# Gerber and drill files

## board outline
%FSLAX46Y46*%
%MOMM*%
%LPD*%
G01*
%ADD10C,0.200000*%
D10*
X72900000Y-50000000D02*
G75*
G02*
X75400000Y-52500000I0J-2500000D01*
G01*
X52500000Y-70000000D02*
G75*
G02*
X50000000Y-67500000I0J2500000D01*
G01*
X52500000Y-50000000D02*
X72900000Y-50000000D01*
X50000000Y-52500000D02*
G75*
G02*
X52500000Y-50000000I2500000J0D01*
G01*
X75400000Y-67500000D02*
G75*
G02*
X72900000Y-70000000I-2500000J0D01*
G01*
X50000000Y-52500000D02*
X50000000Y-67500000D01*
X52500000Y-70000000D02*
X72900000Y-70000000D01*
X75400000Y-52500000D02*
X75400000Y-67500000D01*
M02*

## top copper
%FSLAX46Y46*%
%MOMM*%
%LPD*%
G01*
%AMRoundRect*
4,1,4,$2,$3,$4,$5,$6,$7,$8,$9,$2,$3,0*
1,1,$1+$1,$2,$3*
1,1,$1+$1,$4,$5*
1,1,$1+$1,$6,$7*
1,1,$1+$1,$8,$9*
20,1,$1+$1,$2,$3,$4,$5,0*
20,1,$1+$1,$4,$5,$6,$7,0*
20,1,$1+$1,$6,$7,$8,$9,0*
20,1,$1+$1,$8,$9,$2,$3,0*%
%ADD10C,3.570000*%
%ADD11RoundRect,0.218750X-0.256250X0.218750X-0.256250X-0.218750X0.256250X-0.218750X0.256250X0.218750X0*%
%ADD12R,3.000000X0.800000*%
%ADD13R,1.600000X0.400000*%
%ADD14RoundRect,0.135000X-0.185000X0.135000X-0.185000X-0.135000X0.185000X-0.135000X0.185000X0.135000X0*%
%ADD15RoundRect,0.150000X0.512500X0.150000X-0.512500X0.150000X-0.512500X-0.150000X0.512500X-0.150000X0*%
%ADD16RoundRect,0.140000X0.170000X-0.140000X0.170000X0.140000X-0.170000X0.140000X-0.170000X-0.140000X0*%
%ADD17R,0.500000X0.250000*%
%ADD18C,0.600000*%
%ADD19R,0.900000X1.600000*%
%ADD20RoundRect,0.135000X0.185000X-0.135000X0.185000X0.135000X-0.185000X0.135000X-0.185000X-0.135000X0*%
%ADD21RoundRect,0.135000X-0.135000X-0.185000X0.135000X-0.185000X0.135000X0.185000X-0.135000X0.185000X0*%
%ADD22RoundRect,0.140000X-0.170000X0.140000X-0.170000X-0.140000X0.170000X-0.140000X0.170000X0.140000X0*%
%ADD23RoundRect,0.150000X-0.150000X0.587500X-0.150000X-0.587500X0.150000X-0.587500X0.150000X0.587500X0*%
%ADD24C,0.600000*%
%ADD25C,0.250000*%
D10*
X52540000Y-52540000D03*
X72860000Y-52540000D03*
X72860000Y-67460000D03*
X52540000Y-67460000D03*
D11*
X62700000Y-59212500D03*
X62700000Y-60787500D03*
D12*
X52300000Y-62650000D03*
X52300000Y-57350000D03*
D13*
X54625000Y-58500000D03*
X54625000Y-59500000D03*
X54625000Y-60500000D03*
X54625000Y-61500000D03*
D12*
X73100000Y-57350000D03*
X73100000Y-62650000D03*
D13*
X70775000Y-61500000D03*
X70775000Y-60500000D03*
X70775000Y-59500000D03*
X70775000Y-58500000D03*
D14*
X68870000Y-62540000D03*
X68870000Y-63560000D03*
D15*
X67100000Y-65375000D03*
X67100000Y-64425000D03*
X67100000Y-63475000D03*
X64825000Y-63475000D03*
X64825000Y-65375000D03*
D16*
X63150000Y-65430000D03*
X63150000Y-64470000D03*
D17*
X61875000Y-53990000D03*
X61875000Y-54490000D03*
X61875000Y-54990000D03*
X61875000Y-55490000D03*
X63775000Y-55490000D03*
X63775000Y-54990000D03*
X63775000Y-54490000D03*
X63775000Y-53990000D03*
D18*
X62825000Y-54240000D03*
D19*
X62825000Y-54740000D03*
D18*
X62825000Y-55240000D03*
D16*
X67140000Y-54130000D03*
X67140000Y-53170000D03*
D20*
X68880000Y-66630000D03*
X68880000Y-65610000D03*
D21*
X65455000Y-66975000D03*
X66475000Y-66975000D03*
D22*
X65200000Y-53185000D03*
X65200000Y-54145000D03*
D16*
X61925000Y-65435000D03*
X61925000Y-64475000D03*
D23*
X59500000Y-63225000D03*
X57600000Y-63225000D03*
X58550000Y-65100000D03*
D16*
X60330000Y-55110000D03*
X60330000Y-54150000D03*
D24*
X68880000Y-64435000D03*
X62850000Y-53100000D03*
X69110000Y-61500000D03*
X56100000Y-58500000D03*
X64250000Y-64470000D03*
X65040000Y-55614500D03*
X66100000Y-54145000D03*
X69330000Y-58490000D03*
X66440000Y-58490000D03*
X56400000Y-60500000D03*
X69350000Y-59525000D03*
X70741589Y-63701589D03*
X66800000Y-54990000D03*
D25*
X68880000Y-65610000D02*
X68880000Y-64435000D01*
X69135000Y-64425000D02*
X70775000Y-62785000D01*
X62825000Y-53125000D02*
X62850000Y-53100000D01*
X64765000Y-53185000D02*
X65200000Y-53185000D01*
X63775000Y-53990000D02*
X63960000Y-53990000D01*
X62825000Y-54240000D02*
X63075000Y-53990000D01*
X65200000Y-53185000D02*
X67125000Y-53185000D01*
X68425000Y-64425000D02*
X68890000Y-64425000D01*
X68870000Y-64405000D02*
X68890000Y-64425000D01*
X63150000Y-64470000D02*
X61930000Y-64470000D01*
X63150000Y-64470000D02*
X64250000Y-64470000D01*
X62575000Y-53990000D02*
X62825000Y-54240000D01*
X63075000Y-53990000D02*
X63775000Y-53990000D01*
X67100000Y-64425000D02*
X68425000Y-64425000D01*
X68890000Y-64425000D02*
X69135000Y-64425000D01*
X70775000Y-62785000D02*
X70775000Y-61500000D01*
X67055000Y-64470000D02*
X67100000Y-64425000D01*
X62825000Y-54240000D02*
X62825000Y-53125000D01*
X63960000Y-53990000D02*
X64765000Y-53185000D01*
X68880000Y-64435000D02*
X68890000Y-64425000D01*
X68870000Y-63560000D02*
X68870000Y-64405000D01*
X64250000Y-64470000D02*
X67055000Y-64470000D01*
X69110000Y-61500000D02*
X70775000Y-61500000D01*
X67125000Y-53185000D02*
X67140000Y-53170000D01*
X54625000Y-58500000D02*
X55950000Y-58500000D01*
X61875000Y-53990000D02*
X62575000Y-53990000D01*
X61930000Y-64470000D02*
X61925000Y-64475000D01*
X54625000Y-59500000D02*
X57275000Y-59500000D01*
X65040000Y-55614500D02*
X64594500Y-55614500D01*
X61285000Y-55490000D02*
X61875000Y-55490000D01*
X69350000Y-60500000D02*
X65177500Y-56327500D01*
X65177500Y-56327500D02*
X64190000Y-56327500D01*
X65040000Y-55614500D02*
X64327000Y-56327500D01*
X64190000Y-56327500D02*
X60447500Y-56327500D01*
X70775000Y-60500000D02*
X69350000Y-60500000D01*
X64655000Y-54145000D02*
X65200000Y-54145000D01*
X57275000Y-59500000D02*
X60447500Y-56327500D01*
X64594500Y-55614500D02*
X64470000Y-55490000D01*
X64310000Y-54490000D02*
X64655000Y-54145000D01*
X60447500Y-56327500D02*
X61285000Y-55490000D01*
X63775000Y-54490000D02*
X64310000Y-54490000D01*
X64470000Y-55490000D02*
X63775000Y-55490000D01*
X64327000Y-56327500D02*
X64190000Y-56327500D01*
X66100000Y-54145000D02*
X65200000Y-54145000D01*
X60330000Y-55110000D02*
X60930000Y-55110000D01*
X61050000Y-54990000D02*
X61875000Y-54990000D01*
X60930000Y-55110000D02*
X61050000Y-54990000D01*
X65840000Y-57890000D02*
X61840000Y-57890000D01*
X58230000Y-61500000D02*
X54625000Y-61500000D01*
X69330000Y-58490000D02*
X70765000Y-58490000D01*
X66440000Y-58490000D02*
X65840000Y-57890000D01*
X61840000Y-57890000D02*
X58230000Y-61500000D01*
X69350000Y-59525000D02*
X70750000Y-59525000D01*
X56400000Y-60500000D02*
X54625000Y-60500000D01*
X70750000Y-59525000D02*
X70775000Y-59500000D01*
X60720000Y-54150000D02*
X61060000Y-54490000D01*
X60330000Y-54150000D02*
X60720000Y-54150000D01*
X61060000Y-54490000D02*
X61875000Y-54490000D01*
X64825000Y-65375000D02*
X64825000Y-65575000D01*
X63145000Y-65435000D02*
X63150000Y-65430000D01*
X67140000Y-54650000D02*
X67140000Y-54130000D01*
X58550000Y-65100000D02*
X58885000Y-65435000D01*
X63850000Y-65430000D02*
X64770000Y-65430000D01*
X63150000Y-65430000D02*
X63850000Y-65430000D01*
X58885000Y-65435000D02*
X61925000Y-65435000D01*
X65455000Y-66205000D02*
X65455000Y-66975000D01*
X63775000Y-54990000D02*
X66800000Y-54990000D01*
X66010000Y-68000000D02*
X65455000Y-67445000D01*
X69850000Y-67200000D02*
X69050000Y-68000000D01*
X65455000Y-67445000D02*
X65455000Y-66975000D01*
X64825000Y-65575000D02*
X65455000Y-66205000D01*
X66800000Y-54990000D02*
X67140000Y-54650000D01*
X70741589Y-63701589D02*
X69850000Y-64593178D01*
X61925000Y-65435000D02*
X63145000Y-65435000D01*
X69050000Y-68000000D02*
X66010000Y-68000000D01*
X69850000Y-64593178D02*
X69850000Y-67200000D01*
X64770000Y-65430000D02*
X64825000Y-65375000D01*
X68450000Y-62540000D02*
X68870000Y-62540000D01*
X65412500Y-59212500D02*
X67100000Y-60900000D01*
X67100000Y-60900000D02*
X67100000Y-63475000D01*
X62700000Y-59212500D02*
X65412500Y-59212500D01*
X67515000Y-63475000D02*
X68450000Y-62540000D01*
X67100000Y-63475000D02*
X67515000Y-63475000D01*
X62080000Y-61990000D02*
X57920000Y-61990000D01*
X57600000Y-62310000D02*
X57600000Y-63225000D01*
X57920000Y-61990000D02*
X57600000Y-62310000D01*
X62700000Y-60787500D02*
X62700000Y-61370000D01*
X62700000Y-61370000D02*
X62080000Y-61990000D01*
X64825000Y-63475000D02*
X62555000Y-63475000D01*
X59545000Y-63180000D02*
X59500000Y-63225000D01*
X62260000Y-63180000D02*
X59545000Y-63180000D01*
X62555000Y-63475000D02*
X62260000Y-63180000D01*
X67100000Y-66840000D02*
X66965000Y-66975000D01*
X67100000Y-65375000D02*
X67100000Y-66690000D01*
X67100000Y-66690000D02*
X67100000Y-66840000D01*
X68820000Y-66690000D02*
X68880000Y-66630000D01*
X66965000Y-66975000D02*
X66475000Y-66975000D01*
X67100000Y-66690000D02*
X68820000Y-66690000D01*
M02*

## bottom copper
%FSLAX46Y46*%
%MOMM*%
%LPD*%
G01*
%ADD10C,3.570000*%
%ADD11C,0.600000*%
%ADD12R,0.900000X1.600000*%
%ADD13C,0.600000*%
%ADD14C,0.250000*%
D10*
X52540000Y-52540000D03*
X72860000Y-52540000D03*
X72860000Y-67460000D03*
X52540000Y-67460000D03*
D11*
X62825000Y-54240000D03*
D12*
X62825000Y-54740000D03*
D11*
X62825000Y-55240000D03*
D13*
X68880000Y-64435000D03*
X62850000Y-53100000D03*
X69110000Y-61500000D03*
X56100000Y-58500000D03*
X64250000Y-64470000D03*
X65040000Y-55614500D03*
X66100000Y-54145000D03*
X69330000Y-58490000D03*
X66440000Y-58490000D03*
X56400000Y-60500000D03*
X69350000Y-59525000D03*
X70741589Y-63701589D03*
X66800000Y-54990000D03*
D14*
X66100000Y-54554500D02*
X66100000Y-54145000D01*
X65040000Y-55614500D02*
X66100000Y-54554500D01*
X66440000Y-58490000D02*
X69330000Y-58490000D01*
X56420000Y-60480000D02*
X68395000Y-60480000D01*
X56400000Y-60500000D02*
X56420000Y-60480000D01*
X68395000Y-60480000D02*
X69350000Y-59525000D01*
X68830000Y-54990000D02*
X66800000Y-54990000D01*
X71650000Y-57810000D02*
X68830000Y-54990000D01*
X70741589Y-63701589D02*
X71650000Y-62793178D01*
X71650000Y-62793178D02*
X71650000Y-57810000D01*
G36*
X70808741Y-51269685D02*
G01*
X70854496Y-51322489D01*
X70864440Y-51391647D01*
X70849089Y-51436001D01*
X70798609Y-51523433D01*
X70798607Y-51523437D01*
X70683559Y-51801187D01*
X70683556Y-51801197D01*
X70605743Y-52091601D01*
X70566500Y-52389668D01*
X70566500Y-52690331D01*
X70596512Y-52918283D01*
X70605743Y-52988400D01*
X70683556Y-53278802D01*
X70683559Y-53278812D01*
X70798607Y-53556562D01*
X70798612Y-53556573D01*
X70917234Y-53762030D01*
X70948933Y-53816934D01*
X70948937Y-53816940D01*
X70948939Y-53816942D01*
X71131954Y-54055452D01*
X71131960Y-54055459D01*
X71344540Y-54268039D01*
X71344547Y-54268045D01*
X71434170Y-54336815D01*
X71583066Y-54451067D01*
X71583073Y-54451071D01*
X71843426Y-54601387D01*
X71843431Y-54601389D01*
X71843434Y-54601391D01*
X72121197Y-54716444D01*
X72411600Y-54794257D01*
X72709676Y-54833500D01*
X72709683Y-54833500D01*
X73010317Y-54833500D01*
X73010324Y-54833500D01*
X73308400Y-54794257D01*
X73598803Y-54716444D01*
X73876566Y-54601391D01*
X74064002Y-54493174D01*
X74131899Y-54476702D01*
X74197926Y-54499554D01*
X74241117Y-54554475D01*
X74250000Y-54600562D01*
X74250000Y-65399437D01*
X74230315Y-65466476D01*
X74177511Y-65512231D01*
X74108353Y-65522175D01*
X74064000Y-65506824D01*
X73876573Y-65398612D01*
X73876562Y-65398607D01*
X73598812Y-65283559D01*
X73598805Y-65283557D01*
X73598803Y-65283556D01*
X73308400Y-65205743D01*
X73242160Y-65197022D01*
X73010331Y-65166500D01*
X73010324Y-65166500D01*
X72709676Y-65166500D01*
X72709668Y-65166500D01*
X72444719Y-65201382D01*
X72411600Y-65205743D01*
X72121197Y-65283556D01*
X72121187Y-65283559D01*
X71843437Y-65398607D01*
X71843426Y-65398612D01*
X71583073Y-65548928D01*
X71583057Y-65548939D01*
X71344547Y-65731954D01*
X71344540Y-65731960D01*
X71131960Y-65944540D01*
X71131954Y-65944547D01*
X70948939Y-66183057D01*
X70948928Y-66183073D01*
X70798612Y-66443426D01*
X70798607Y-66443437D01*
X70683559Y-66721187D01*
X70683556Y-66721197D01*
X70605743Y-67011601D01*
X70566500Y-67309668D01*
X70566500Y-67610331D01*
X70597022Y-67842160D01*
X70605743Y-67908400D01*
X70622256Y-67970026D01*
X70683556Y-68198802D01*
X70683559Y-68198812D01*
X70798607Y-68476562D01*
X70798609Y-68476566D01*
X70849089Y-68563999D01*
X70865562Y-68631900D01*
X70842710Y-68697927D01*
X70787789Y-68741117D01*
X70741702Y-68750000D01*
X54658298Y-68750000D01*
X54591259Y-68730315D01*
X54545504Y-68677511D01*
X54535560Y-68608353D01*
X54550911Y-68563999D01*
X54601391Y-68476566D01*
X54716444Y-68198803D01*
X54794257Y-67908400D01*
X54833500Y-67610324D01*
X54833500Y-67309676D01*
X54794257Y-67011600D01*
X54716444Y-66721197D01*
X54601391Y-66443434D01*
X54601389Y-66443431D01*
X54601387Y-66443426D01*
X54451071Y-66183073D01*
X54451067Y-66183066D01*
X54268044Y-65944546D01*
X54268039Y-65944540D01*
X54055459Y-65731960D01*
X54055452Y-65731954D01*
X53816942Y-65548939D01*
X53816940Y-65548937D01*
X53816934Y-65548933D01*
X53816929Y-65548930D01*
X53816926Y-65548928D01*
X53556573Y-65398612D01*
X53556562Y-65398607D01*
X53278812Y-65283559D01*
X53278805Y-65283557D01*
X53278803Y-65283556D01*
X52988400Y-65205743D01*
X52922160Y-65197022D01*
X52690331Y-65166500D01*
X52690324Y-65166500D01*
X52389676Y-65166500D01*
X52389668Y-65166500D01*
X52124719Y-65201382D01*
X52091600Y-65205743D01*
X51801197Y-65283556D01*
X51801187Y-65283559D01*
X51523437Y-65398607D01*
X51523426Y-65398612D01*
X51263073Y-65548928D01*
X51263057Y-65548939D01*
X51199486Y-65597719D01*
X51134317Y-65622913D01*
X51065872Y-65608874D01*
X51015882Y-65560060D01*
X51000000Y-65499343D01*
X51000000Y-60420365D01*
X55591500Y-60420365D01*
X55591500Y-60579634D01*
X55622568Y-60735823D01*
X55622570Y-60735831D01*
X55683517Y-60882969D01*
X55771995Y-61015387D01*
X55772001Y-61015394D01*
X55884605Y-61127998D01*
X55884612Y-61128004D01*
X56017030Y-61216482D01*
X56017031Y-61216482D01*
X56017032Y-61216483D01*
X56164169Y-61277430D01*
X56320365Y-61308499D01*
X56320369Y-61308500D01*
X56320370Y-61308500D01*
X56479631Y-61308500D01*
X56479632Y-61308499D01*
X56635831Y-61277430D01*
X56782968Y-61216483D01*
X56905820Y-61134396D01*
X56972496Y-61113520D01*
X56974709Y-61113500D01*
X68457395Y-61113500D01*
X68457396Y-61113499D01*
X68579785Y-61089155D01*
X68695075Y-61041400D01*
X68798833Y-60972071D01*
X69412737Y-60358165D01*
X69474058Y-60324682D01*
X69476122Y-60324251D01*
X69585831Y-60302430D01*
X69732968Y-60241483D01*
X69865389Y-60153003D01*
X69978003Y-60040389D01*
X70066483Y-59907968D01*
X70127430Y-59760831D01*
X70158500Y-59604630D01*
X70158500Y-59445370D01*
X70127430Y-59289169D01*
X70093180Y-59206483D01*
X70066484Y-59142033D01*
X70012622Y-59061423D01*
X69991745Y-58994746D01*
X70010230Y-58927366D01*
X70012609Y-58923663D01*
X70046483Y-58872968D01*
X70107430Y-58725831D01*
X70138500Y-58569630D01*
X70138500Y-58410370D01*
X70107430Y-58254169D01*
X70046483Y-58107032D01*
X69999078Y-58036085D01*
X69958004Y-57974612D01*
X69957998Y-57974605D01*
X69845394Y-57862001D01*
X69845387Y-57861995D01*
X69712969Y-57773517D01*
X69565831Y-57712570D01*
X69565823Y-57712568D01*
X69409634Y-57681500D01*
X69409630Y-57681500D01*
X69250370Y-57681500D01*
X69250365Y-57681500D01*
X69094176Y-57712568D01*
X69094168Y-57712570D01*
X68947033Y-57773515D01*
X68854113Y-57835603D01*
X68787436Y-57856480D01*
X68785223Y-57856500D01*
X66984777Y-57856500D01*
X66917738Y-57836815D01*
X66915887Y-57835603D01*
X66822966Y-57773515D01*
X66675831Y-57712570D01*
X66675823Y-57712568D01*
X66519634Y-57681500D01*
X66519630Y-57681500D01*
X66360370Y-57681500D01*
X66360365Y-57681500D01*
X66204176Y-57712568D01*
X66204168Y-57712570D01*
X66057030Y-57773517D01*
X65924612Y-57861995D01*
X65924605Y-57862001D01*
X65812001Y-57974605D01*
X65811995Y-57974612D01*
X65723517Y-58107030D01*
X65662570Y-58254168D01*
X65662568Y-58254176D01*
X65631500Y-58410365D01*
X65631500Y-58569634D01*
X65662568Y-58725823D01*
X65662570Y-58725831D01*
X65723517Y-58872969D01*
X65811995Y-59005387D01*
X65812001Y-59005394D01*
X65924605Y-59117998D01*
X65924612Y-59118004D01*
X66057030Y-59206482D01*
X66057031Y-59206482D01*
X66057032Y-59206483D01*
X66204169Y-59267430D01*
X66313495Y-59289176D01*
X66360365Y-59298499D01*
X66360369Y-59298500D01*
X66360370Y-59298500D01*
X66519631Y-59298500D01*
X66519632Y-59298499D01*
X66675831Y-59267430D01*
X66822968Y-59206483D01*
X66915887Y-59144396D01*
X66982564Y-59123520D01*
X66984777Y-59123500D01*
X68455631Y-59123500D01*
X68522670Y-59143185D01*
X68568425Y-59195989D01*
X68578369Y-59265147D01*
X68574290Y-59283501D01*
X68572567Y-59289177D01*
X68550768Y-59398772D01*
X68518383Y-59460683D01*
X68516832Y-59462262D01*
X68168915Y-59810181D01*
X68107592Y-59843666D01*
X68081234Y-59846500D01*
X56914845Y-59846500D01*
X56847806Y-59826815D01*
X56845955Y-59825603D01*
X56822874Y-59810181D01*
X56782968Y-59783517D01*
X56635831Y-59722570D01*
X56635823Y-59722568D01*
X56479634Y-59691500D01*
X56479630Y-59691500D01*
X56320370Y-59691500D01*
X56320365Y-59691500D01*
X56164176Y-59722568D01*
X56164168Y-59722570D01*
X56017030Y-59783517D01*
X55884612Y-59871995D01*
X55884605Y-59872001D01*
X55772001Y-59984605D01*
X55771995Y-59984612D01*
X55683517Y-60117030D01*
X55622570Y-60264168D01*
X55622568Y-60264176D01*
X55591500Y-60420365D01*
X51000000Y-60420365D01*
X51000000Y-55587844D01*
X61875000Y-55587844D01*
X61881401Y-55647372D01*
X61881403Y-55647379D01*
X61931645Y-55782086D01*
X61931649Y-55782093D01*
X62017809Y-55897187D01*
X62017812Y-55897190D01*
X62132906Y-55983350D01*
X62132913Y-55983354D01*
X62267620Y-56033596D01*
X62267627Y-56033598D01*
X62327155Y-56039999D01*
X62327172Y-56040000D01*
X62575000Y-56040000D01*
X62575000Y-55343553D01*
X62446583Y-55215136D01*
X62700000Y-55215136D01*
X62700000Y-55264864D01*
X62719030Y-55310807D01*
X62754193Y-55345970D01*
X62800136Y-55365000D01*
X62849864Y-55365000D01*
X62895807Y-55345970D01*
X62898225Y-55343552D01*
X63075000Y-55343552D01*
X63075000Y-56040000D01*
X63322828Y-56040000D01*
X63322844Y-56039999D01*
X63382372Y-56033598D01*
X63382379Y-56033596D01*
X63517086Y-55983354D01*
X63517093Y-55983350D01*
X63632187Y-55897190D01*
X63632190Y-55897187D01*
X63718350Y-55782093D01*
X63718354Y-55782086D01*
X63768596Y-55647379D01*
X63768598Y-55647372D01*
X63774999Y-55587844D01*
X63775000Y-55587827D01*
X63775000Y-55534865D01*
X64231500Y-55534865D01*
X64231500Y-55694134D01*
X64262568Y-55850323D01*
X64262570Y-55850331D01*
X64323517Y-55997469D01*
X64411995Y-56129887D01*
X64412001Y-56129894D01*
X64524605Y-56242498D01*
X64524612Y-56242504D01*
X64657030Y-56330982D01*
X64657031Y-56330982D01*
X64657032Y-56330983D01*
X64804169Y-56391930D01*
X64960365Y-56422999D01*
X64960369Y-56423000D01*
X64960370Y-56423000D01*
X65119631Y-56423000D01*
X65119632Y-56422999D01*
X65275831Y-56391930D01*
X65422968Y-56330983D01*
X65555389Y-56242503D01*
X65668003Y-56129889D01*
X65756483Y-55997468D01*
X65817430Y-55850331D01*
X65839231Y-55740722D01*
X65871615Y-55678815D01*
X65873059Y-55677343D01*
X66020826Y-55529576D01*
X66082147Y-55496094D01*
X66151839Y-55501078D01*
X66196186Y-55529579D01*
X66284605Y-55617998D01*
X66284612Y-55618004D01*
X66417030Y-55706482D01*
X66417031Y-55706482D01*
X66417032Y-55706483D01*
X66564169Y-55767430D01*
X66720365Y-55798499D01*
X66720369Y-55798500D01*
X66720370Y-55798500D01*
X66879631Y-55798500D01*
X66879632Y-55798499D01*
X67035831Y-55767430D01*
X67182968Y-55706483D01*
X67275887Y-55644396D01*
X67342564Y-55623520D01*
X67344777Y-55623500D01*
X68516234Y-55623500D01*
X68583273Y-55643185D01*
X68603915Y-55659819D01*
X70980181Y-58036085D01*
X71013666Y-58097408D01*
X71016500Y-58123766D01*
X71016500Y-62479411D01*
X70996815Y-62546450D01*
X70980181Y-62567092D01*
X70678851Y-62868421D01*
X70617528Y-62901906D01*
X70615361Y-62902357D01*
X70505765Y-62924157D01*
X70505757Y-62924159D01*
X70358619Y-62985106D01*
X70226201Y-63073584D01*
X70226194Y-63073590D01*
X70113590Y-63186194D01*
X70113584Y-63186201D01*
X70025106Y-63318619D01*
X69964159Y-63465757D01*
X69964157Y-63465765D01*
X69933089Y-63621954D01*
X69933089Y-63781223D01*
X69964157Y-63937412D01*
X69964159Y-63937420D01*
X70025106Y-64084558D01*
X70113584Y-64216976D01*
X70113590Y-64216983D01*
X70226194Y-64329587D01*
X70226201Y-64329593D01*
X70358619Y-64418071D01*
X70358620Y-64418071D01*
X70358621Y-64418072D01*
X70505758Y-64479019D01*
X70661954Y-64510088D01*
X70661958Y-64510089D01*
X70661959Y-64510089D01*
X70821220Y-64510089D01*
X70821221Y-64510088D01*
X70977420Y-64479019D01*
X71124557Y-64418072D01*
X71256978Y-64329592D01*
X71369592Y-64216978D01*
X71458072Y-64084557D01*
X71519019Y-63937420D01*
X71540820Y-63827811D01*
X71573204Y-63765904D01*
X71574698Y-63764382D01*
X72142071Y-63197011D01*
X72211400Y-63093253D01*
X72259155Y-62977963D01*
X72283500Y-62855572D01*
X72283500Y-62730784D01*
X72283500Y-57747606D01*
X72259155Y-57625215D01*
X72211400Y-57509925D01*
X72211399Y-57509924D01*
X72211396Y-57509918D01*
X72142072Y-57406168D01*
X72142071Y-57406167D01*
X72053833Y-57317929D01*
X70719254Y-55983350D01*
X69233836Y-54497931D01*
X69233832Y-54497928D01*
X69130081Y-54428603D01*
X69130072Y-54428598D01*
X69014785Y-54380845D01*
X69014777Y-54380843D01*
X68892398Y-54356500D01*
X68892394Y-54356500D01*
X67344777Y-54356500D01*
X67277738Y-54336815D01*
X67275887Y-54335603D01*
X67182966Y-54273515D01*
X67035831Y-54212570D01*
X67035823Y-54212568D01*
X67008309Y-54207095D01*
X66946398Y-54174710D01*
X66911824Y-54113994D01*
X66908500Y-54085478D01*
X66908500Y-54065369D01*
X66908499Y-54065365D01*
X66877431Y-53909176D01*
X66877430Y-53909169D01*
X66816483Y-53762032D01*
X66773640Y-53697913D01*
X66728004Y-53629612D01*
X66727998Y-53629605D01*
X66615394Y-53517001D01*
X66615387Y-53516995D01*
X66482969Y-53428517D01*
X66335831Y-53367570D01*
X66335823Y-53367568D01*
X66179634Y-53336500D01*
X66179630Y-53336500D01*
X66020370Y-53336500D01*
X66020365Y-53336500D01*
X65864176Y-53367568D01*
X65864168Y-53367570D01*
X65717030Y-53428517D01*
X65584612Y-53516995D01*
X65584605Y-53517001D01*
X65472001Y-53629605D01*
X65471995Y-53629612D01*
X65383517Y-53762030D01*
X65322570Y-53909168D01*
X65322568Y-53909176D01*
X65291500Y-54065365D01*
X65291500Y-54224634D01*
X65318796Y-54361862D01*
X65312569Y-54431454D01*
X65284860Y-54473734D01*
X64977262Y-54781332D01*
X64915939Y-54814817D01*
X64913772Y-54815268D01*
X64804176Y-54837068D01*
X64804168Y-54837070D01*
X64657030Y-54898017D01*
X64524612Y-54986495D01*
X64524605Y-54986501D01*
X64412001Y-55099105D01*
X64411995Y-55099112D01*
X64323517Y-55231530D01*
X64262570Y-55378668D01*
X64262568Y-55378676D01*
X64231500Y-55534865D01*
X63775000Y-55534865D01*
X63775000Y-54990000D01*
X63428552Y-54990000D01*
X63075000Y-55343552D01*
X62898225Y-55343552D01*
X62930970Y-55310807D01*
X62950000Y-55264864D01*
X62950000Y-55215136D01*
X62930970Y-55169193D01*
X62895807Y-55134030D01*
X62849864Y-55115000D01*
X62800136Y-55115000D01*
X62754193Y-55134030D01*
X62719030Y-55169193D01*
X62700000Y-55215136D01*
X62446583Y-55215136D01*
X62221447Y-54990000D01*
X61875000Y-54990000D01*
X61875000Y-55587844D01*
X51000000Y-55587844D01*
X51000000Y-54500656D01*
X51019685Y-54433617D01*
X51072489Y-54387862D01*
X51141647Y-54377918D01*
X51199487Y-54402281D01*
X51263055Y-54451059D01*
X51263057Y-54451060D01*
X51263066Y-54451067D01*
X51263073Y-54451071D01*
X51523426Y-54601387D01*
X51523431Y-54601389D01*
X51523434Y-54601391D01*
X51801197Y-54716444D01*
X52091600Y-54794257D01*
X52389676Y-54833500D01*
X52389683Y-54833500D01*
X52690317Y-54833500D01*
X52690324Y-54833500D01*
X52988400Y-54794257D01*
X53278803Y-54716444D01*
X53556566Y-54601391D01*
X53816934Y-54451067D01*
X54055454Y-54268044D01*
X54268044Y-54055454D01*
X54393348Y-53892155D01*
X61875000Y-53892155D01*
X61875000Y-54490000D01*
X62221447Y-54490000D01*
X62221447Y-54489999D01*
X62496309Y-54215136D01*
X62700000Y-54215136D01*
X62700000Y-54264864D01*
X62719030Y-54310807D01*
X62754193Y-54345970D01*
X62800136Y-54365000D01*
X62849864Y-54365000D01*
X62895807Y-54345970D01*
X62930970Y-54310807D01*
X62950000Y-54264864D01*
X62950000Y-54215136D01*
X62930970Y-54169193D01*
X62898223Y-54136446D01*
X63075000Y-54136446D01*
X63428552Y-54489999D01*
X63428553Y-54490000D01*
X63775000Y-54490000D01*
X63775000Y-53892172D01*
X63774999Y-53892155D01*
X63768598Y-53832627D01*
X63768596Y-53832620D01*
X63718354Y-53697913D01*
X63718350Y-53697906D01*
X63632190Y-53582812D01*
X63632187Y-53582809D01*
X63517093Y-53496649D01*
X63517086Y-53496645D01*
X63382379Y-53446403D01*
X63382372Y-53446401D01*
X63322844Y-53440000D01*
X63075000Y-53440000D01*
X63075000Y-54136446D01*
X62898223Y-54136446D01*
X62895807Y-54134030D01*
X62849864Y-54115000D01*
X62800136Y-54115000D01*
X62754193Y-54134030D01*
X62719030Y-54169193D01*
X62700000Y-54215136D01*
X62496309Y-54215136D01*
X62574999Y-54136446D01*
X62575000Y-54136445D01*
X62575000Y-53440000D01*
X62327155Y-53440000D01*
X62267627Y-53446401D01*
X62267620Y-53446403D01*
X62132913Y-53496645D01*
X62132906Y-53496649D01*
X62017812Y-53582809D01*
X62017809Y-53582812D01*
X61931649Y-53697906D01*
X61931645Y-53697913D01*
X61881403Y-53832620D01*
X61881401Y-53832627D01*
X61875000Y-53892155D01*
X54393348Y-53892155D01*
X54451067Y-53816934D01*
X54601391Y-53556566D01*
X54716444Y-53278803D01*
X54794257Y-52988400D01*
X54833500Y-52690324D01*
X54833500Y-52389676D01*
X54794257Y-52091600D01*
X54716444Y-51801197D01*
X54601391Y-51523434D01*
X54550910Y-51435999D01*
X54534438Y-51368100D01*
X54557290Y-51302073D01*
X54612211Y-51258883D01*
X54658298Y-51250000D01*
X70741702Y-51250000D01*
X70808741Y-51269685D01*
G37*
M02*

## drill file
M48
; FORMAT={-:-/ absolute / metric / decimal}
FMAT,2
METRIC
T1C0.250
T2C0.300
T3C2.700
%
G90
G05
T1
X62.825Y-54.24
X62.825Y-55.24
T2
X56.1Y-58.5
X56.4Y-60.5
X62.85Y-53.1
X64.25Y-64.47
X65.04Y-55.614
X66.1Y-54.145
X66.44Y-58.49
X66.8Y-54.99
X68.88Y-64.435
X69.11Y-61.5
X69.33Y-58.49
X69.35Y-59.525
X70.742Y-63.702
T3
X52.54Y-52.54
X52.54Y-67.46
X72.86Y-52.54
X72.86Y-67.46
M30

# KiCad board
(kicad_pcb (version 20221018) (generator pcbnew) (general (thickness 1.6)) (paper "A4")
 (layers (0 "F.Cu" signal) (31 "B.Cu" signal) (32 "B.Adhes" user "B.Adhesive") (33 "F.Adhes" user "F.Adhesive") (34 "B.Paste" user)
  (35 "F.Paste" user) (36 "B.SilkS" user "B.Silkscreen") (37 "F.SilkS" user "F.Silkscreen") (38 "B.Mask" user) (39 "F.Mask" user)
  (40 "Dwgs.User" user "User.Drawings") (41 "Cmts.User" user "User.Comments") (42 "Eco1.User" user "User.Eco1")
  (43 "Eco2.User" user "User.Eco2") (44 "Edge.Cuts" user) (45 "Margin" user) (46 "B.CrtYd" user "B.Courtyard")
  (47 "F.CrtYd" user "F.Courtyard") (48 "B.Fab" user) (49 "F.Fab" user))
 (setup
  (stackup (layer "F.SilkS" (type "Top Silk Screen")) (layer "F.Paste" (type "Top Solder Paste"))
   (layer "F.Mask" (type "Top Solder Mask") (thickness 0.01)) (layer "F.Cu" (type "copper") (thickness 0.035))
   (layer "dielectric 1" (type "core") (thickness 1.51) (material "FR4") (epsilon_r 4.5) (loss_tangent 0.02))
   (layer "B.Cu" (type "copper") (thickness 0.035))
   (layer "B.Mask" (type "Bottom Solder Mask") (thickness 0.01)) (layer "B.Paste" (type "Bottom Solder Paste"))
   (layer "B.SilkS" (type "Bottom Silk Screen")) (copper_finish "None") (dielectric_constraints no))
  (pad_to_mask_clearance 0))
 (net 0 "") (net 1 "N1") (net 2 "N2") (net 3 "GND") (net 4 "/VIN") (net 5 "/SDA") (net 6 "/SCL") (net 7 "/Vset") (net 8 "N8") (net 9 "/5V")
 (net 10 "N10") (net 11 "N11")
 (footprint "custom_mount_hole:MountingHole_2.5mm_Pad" (layer "F.Cu") (at 52.54 52.54)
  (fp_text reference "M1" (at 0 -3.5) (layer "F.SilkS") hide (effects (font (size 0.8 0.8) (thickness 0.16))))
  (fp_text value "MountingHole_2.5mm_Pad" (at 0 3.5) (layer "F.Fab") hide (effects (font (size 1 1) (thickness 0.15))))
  (pad "~" thru_hole circle (at 0 0) (size 3.57 3.57) (drill 2.7) (layers "*.Cu" "*.Mask")))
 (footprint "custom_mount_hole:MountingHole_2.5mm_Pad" (layer "F.Cu") (at 72.86 52.54)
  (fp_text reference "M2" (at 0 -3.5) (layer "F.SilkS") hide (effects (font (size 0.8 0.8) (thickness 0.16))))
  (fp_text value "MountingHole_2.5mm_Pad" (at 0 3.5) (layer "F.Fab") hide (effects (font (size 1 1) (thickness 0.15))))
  (pad "~" thru_hole circle (at 0 0) (size 3.57 3.57) (drill 2.7) (layers "*.Cu" "*.Mask")))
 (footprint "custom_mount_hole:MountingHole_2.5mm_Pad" (layer "F.Cu") (at 72.86 67.46)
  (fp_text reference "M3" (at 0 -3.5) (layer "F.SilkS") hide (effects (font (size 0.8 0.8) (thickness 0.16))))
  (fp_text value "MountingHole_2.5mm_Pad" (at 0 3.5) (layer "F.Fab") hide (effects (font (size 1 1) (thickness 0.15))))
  (pad "~" thru_hole circle (at 0 0) (size 3.57 3.57) (drill 2.7) (layers "*.Cu" "*.Mask")))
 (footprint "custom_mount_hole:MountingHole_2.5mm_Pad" (layer "F.Cu") (at 52.54 67.46)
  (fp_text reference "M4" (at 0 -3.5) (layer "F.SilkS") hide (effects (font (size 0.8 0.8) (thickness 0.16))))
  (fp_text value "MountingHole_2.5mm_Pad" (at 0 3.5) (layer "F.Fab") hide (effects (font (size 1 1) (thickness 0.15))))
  (pad "~" thru_hole circle (at 0 0) (size 3.57 3.57) (drill 2.7) (layers "*.Cu" "*.Mask")))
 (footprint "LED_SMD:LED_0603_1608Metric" (layer "F.Cu") (at 62.7 60 -90)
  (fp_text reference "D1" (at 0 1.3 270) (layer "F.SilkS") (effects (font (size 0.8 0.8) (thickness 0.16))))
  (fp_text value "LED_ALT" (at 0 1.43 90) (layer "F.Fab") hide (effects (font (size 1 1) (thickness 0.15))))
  (pad "1" smd roundrect (at -0.7875 0 270) (size 0.875 0.95) (layers "F.Cu" "F.Paste" "F.Mask") (roundrect_rratio 0.25) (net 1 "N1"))
  (pad "2" smd roundrect (at 0.7875 0 270) (size 0.875 0.95) (layers "F.Cu" "F.Paste" "F.Mask") (roundrect_rratio 0.25) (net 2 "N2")))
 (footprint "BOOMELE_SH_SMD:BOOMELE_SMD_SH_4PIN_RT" (layer "F.Cu") (at 52.78 60 90)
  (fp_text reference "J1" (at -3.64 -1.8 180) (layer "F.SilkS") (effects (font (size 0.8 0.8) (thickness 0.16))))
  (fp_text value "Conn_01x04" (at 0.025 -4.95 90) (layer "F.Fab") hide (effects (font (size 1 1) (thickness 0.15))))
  (pad "" smd rect (at -2.65 -0.48 270) (size 0.8 3) (layers "F.Cu" "F.Paste" "F.Mask"))
  (pad "" smd rect (at 2.65 -0.48 270) (size 0.8 3) (layers "F.Cu" "F.Paste" "F.Mask"))
  (pad "1" smd rect (at 1.5 1.845 270) (size 0.4 1.6) (layers "F.Cu" "F.Paste" "F.Mask") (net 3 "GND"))
  (pad "2" smd rect (at 0.5 1.845 270) (size 0.4 1.6) (layers "F.Cu" "F.Paste" "F.Mask") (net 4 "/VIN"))
  (pad "3" smd rect (at -0.5 1.845 270) (size 0.4 1.6) (layers "F.Cu" "F.Paste" "F.Mask") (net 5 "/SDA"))
  (pad "4" smd rect (at -1.5 1.845 270) (size 0.4 1.6) (layers "F.Cu" "F.Paste" "F.Mask") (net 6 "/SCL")))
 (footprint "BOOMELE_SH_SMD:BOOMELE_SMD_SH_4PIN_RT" (layer "F.Cu") (at 72.62 60 -90)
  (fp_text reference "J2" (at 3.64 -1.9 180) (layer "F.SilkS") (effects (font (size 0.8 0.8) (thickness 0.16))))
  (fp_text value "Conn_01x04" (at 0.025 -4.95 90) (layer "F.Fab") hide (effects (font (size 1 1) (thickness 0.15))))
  (pad "" smd rect (at -2.65 -0.48 90) (size 0.8 3) (layers "F.Cu" "F.Paste" "F.Mask"))
  (pad "" smd rect (at 2.65 -0.48 90) (size 0.8 3) (layers "F.Cu" "F.Paste" "F.Mask"))
  (pad "1" smd rect (at 1.5 1.845 90) (size 0.4 1.6) (layers "F.Cu" "F.Paste" "F.Mask") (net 3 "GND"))
  (pad "2" smd rect (at 0.5 1.845 90) (size 0.4 1.6) (layers "F.Cu" "F.Paste" "F.Mask") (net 4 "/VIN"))
  (pad "3" smd rect (at -0.5 1.845 90) (size 0.4 1.6) (layers "F.Cu" "F.Paste" "F.Mask") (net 5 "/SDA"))
  (pad "4" smd rect (at -1.5 1.845 90) (size 0.4 1.6) (layers "F.Cu" "F.Paste" "F.Mask") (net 6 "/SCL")))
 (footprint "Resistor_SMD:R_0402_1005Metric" (layer "F.Cu") (at 68.87 63.05 -90)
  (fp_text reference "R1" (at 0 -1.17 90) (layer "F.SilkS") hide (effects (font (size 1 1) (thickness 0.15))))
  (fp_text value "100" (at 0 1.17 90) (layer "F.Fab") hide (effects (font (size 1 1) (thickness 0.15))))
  (pad "1" smd roundrect (at -0.51 0 270) (size 0.54 0.64) (layers "F.Cu" "F.Paste" "F.Mask") (roundrect_rratio 0.25) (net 1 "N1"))
  (pad "2" smd roundrect (at 0.51 0 270) (size 0.54 0.64) (layers "F.Cu" "F.Paste" "F.Mask") (roundrect_rratio 0.25) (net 3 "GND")))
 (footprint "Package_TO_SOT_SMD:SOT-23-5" (layer "F.Cu") (at 65.9625 64.425 180)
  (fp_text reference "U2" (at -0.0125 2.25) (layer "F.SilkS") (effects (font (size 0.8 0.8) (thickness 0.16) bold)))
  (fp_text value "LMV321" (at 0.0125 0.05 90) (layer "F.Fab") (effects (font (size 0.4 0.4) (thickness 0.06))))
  (pad "1" smd roundrect (at -1.1375 -0.95 180) (size 1.325 0.6) (layers "F.Cu" "F.Paste" "F.Mask") (roundrect_rratio 0.25) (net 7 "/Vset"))
  (pad "2" smd roundrect (at -1.1375 0 180) (size 1.325 0.6) (layers "F.Cu" "F.Paste" "F.Mask") (roundrect_rratio 0.25) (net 3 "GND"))
  (pad "3" smd roundrect (at -1.1375 0.95 180) (size 1.325 0.6) (layers "F.Cu" "F.Paste" "F.Mask") (roundrect_rratio 0.25) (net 1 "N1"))
  (pad "4" smd roundrect (at 1.1375 0.95 180) (size 1.325 0.6) (layers "F.Cu" "F.Paste" "F.Mask") (roundrect_rratio 0.25) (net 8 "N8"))
  (pad "5" smd roundrect (at 1.1375 -0.95 180) (size 1.325 0.6) (layers "F.Cu" "F.Paste" "F.Mask") (roundrect_rratio 0.25) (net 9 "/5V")))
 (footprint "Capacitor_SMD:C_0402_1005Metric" (layer "F.Cu") (at 63.15 64.95 90)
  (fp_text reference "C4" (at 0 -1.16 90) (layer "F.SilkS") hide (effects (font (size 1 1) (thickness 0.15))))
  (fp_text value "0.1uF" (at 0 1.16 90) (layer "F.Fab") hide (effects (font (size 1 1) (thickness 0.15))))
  (pad "1" smd roundrect (at -0.48 0 90) (size 0.56 0.62) (layers "F.Cu" "F.Paste" "F.Mask") (roundrect_rratio 0.25) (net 9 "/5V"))
  (pad "2" smd roundrect (at 0.48 0 90) (size 0.56 0.62) (layers "F.Cu" "F.Paste" "F.Mask") (roundrect_rratio 0.25) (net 3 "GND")))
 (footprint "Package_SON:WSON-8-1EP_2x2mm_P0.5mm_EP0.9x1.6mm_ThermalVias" (layer "F.Cu") (at 62.825 54.74)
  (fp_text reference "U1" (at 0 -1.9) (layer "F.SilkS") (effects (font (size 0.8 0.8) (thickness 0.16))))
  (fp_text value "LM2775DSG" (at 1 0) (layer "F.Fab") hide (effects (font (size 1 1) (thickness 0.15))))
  (pad "" smd rect (at 0 -0.4) (size 0.75 0.65) (layers "F.Paste"))
  (pad "" smd rect (at 0 0.4) (size 0.75 0.65) (layers "F.Paste"))
  (pad "1" smd rect (at -0.95 -0.75) (size 0.5 0.25) (layers "F.Cu" "F.Paste" "F.Mask") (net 3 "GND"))
  (pad "2" smd rect (at -0.95 -0.25) (size 0.5 0.25) (layers "F.Cu" "F.Paste" "F.Mask") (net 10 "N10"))
  (pad "3" smd rect (at -0.95 0.25) (size 0.5 0.25) (layers "F.Cu" "F.Paste" "F.Mask") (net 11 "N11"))
  (pad "4" smd rect (at -0.95 0.75) (size 0.5 0.25) (layers "F.Cu" "F.Paste" "F.Mask") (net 4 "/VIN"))
  (pad "5" smd rect (at 0.95 0.75) (size 0.5 0.25) (layers "F.Cu" "F.Paste" "F.Mask") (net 4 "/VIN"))
  (pad "6" smd rect (at 0.95 0.25) (size 0.5 0.25) (layers "F.Cu" "F.Paste" "F.Mask") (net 9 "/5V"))
  (pad "7" smd rect (at 0.95 -0.25) (size 0.5 0.25) (layers "F.Cu" "F.Paste" "F.Mask") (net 4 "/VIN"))
  (pad "8" smd rect (at 0.95 -0.75) (size 0.5 0.25) (layers "F.Cu" "F.Paste" "F.Mask") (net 3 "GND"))
  (pad "9" thru_hole circle (at 0 -0.5) (size 0.6 0.6) (drill 0.25) (layers "*.Cu") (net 3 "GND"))
  (pad "9" smd rect (at 0 0) (size 0.9 1.6) (layers "F.Cu" "F.Mask") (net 3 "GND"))
  (pad "9" smd rect (at 0 0) (size 0.9 1.6) (layers "B.Cu") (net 3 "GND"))
  (pad "9" thru_hole circle (at 0 0.5) (size 0.6 0.6) (drill 0.25) (layers "*.Cu") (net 3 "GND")))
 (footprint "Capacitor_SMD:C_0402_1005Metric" (layer "F.Cu") (at 67.14 53.65 90)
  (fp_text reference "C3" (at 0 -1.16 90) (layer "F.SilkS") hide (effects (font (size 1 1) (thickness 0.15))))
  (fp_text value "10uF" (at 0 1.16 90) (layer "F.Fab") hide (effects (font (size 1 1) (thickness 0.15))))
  (pad "1" smd roundrect (at -0.48 0 90) (size 0.56 0.62) (layers "F.Cu" "F.Paste" "F.Mask") (roundrect_rratio 0.25) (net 9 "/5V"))
  (pad "2" smd roundrect (at 0.48 0 90) (size 0.56 0.62) (layers "F.Cu" "F.Paste" "F.Mask") (roundrect_rratio 0.25) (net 3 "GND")))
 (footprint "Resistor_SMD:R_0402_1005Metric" (layer "F.Cu") (at 68.88 66.12 90)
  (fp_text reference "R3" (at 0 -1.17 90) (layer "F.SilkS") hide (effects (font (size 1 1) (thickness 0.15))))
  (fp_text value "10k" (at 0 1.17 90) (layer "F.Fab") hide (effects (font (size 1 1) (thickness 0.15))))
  (pad "1" smd roundrect (at -0.51 0 90) (size 0.54 0.64) (layers "F.Cu" "F.Paste" "F.Mask") (roundrect_rratio 0.25) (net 7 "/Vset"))
  (pad "2" smd roundrect (at 0.51 0 90) (size 0.54 0.64) (layers "F.Cu" "F.Paste" "F.Mask") (roundrect_rratio 0.25) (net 3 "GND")))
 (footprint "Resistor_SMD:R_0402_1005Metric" (layer "F.Cu") (at 65.965 66.975)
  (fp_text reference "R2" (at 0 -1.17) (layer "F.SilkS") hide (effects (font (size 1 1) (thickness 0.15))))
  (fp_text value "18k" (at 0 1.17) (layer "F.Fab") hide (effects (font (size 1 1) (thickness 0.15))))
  (pad "1" smd roundrect (at -0.51 0) (size 0.54 0.64) (layers "F.Cu" "F.Paste" "F.Mask") (roundrect_rratio 0.25) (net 9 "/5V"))
  (pad "2" smd roundrect (at 0.51 0) (size 0.54 0.64) (layers "F.Cu" "F.Paste" "F.Mask") (roundrect_rratio 0.25) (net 7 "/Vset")))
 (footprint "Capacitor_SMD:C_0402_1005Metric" (layer "F.Cu") (at 65.2 53.665 -90)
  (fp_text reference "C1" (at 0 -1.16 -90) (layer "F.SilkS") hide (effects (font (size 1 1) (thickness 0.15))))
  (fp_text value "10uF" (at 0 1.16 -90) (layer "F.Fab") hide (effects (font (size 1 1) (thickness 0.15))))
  (pad "1" smd roundrect (at -0.48 0 270) (size 0.56 0.62) (layers "F.Cu" "F.Paste" "F.Mask") (roundrect_rratio 0.25) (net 3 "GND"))
  (pad "2" smd roundrect (at 0.48 0 270) (size 0.56 0.62) (layers "F.Cu" "F.Paste" "F.Mask") (roundrect_rratio 0.25) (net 4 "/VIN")))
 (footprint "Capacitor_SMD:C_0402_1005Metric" (layer "F.Cu") (at 61.925 64.955 90)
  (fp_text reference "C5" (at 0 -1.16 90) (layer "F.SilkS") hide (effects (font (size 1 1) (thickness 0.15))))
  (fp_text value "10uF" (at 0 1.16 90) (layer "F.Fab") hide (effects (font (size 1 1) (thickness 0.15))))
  (pad "1" smd roundrect (at -0.48 0 90) (size 0.56 0.62) (layers "F.Cu" "F.Paste" "F.Mask") (roundrect_rratio 0.25) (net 9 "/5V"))
  (pad "2" smd roundrect (at 0.48 0 90) (size 0.56 0.62) (layers "F.Cu" "F.Paste" "F.Mask") (roundrect_rratio 0.25) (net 3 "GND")))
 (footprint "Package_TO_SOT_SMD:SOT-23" (layer "F.Cu") (at 58.55 64.1625 -90)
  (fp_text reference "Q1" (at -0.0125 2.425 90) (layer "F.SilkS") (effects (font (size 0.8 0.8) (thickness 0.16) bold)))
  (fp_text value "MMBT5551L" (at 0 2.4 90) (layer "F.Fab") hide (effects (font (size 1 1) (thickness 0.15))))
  (pad "1" smd roundrect (at -0.9375 -0.95 270) (size 1.475 0.6) (layers "F.Cu" "F.Paste" "F.Mask") (roundrect_rratio 0.25) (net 8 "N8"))
  (pad "2" smd roundrect (at -0.9375 0.95 270) (size 1.475 0.6) (layers "F.Cu" "F.Paste" "F.Mask") (roundrect_rratio 0.25) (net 2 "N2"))
  (pad "3" smd roundrect (at 0.9375 0 270) (size 1.475 0.6) (layers "F.Cu" "F.Paste" "F.Mask") (roundrect_rratio 0.25) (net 9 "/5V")))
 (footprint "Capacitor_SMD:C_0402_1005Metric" (layer "F.Cu") (at 60.33 54.63 90)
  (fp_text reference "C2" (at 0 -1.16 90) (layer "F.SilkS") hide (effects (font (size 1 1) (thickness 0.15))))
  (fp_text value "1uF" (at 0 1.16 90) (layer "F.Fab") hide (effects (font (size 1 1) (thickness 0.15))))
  (pad "1" smd roundrect (at -0.48 0 90) (size 0.56 0.62) (layers "F.Cu" "F.Paste" "F.Mask") (roundrect_rratio 0.25) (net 11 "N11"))
  (pad "2" smd roundrect (at 0.48 0 90) (size 0.56 0.62) (layers "F.Cu" "F.Paste" "F.Mask") (roundrect_rratio 0.25) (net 10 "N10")))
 (gr_arc (start 72.9 50) (mid 74.667767 50.732233) (end 75.4 52.5) (stroke (width 0.2) (type solid)) (layer "Edge.Cuts"))
 (gr_arc (start 52.5 70) (mid 50.732233 69.267767) (end 50 67.5) (stroke (width 0.2) (type solid)) (layer "Edge.Cuts"))
 (gr_line (start 52.5 50) (end 72.9 50) (stroke (width 0.2) (type solid)) (layer "Edge.Cuts"))
 (gr_arc (start 50 52.5) (mid 50.732233 50.732233) (end 52.5 50) (stroke (width 0.2) (type solid)) (layer "Edge.Cuts"))
 (gr_arc (start 75.4 67.5) (mid 74.667767 69.267767) (end 72.9 70) (stroke (width 0.2) (type solid)) (layer "Edge.Cuts"))
 (gr_line (start 50 52.5) (end 50 67.5) (stroke (width 0.2) (type solid)) (layer "Edge.Cuts"))
 (gr_line (start 52.5 70) (end 72.9 70) (stroke (width 0.2) (type solid)) (layer "Edge.Cuts"))
 (gr_line (start 75.4 52.5) (end 75.4 67.5) (stroke (width 0.2) (type solid)) (layer "Edge.Cuts"))
 (segment (start 68.88 65.61) (end 68.88 64.435) (width 0.25) (layer "F.Cu") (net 3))
 (segment (start 69.135 64.425) (end 70.775 62.785) (width 0.25) (layer "F.Cu") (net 3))
 (segment (start 62.825 53.125) (end 62.85 53.1) (width 0.25) (layer "F.Cu") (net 3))
 (segment (start 64.765 53.185) (end 65.2 53.185) (width 0.25) (layer "F.Cu") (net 3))
 (segment (start 63.775 53.99) (end 63.96 53.99) (width 0.25) (layer "F.Cu") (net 3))
 (segment (start 62.825 54.24) (end 63.075 53.99) (width 0.25) (layer "F.Cu") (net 3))
 (segment (start 65.2 53.185) (end 67.125 53.185) (width 0.25) (layer "F.Cu") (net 3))
 (segment (start 68.425 64.425) (end 68.89 64.425) (width 0.25) (layer "F.Cu") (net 3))
 (segment (start 68.87 64.405) (end 68.89 64.425) (width 0.25) (layer "F.Cu") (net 3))
 (segment (start 63.15 64.47) (end 61.93 64.47) (width 0.25) (layer "F.Cu") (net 3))
 (segment (start 63.15 64.47) (end 64.25 64.47) (width 0.25) (layer "F.Cu") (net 3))
 (segment (start 62.575 53.99) (end 62.825 54.24) (width 0.25) (layer "F.Cu") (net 3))
 (segment (start 63.075 53.99) (end 63.775 53.99) (width 0.25) (layer "F.Cu") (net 3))
 (segment (start 67.1 64.425) (end 68.425 64.425) (width 0.25) (layer "F.Cu") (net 3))
 (segment (start 68.89 64.425) (end 69.135 64.425) (width 0.25) (layer "F.Cu") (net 3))
 (segment (start 70.775 62.785) (end 70.775 61.5) (width 0.25) (layer "F.Cu") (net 3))
 (segment (start 67.055 64.47) (end 67.1 64.425) (width 0.25) (layer "F.Cu") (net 3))
 (segment (start 62.825 54.24) (end 62.825 53.125) (width 0.25) (layer "F.Cu") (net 3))
 (segment (start 63.96 53.99) (end 64.765 53.185) (width 0.25) (layer "F.Cu") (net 3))
 (segment (start 68.88 64.435) (end 68.89 64.425) (width 0.25) (layer "F.Cu") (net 3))
 (segment (start 68.87 63.56) (end 68.87 64.405) (width 0.25) (layer "F.Cu") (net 3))
 (segment (start 64.25 64.47) (end 67.055 64.47) (width 0.25) (layer "F.Cu") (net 3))
 (segment (start 69.11 61.5) (end 70.775 61.5) (width 0.25) (layer "F.Cu") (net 3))
 (segment (start 67.125 53.185) (end 67.14 53.17) (width 0.25) (layer "F.Cu") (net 3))
 (segment (start 54.625 58.5) (end 55.95 58.5) (width 0.25) (layer "F.Cu") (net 3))
 (segment (start 61.875 53.99) (end 62.575 53.99) (width 0.25) (layer "F.Cu") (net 3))
 (segment (start 61.93 64.47) (end 61.925 64.475) (width 0.25) (layer "F.Cu") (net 3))
 (via (at 68.88 64.435) (size 0.6) (drill 0.3) (layers "F.Cu" "B.Cu") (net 3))
 (via (at 62.85 53.1) (size 0.6) (drill 0.3) (layers "F.Cu" "B.Cu") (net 3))
 (via (at 69.11 61.5) (size 0.6) (drill 0.3) (layers "F.Cu" "B.Cu") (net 3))
 (via (at 56.1 58.5) (size 0.6) (drill 0.3) (layers "F.Cu" "B.Cu") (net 3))
 (via (at 64.25 64.47) (size 0.6) (drill 0.3) (layers "F.Cu" "B.Cu") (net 3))
 (segment (start 54.625 59.5) (end 57.275 59.5) (width 0.25) (layer "F.Cu") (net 4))
 (segment (start 65.04 55.6145) (end 64.5945 55.6145) (width 0.25) (layer "F.Cu") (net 4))
 (segment (start 61.285 55.49) (end 61.875 55.49) (width 0.25) (layer "F.Cu") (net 4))
 (segment (start 69.35 60.5) (end 65.1775 56.3275) (width 0.25) (layer "F.Cu") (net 4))
 (segment (start 65.1775 56.3275) (end 64.19 56.3275) (width 0.25) (layer "F.Cu") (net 4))
 (segment (start 65.04 55.6145) (end 64.327 56.3275) (width 0.25) (layer "F.Cu") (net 4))
 (segment (start 64.19 56.3275) (end 60.4475 56.3275) (width 0.25) (layer "F.Cu") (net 4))
 (segment (start 70.775 60.5) (end 69.35 60.5) (width 0.25) (layer "F.Cu") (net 4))
 (segment (start 64.655 54.145) (end 65.2 54.145) (width 0.25) (layer "F.Cu") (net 4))
 (segment (start 57.275 59.5) (end 60.4475 56.3275) (width 0.25) (layer "F.Cu") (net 4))
 (segment (start 64.5945 55.6145) (end 64.47 55.49) (width 0.25) (layer "F.Cu") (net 4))
 (segment (start 64.31 54.49) (end 64.655 54.145) (width 0.25) (layer "F.Cu") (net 4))
 (segment (start 60.4475 56.3275) (end 61.285 55.49) (width 0.25) (layer "F.Cu") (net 4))
 (segment (start 63.775 54.49) (end 64.31 54.49) (width 0.25) (layer "F.Cu") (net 4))
 (segment (start 64.47 55.49) (end 63.775 55.49) (width 0.25) (layer "F.Cu") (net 4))
 (segment (start 64.327 56.3275) (end 64.19 56.3275) (width 0.25) (layer "F.Cu") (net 4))
 (segment (start 66.1 54.145) (end 65.2 54.145) (width 0.25) (layer "F.Cu") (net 4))
 (via (at 65.04 55.6145) (size 0.6) (drill 0.3) (layers "F.Cu" "B.Cu") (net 4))
 (via (at 66.1 54.145) (size 0.6) (drill 0.3) (layers "F.Cu" "B.Cu") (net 4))
 (segment (start 66.1 54.5545) (end 66.1 54.145) (width 0.25) (layer "B.Cu") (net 4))
 (segment (start 65.04 55.6145) (end 66.1 54.5545) (width 0.25) (layer "B.Cu") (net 4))
 (segment (start 60.33 55.11) (end 60.93 55.11) (width 0.25) (layer "F.Cu") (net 11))
 (segment (start 61.05 54.99) (end 61.875 54.99) (width 0.25) (layer "F.Cu") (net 11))
 (segment (start 60.93 55.11) (end 61.05 54.99) (width 0.25) (layer "F.Cu") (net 11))
 (segment (start 65.84 57.89) (end 61.84 57.89) (width 0.25) (layer "F.Cu") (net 6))
 (segment (start 58.23 61.5) (end 54.625 61.5) (width 0.25) (layer "F.Cu") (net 6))
 (segment (start 69.33 58.49) (end 70.765 58.49) (width 0.25) (layer "F.Cu") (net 6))
 (segment (start 66.44 58.49) (end 65.84 57.89) (width 0.25) (layer "F.Cu") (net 6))
 (segment (start 61.84 57.89) (end 58.23 61.5) (width 0.25) (layer "F.Cu") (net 6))
 (via (at 69.33 58.49) (size 0.6) (drill 0.3) (layers "F.Cu" "B.Cu") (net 6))
 (via (at 66.44 58.49) (size 0.6) (drill 0.3) (layers "F.Cu" "B.Cu") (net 6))
 (segment (start 66.44 58.49) (end 69.33 58.49) (width 0.25) (layer "B.Cu") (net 6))
 (segment (start 69.35 59.525) (end 70.75 59.525) (width 0.25) (layer "F.Cu") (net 5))
 (segment (start 56.4 60.5) (end 54.625 60.5) (width 0.25) (layer "F.Cu") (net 5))
 (segment (start 70.75 59.525) (end 70.775 59.5) (width 0.25) (layer "F.Cu") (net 5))
 (via (at 56.4 60.5) (size 0.6) (drill 0.3) (layers "F.Cu" "B.Cu") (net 5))
 (via (at 69.35 59.525) (size 0.6) (drill 0.3) (layers "F.Cu" "B.Cu") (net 5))
 (segment (start 56.42 60.48) (end 68.395 60.48) (width 0.25) (layer "B.Cu") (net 5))
 (segment (start 56.4 60.5) (end 56.42 60.48) (width 0.25) (layer "B.Cu") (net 5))
 (segment (start 68.395 60.48) (end 69.35 59.525) (width 0.25) (layer "B.Cu") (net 5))
 (segment (start 60.72 54.15) (end 61.06 54.49) (width 0.25) (layer "F.Cu") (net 10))
 (segment (start 60.33 54.15) (end 60.72 54.15) (width 0.25) (layer "F.Cu") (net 10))
 (segment (start 61.06 54.49) (end 61.875 54.49) (width 0.25) (layer "F.Cu") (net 10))
 (segment (start 64.825 65.375) (end 64.825 65.575) (width 0.25) (layer "F.Cu") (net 9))
 (segment (start 63.145 65.435) (end 63.15 65.43) (width 0.25) (layer "F.Cu") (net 9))
 (segment (start 67.14 54.65) (end 67.14 54.13) (width 0.25) (layer "F.Cu") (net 9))
 (segment (start 58.55 65.1) (end 58.885 65.435) (width 0.25) (layer "F.Cu") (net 9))
 (segment (start 63.85 65.43) (end 64.77 65.43) (width 0.25) (layer "F.Cu") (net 9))
 (segment (start 63.15 65.43) (end 63.85 65.43) (width 0.25) (layer "F.Cu") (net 9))
 (segment (start 58.885 65.435) (end 61.925 65.435) (width 0.25) (layer "F.Cu") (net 9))
 (segment (start 65.455 66.205) (end 65.455 66.975) (width 0.25) (layer "F.Cu") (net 9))
 (segment (start 63.775 54.99) (end 66.8 54.99) (width 0.25) (layer "F.Cu") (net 9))
 (segment (start 66.01 68) (end 65.455 67.445) (width 0.25) (layer "F.Cu") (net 9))
 (segment (start 69.85 67.2) (end 69.05 68) (width 0.25) (layer "F.Cu") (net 9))
 (segment (start 65.455 67.445) (end 65.455 66.975) (width 0.25) (layer "F.Cu") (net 9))
 (segment (start 64.825 65.575) (end 65.455 66.205) (width 0.25) (layer "F.Cu") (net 9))
 (segment (start 66.8 54.99) (end 67.14 54.65) (width 0.25) (layer "F.Cu") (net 9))
 (segment (start 70.741589 63.701589) (end 69.85 64.593178) (width 0.25) (layer "F.Cu") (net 9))
 (segment (start 61.925 65.435) (end 63.145 65.435) (width 0.25) (layer "F.Cu") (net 9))
 (segment (start 69.05 68) (end 66.01 68) (width 0.25) (layer "F.Cu") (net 9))
 (segment (start 69.85 64.593178) (end 69.85 67.2) (width 0.25) (layer "F.Cu") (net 9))
 (segment (start 64.77 65.43) (end 64.825 65.375) (width 0.25) (layer "F.Cu") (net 9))
 (via (at 70.741589 63.701589) (size 0.6) (drill 0.3) (layers "F.Cu" "B.Cu") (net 9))
 (via (at 66.8 54.99) (size 0.6) (drill 0.3) (layers "F.Cu" "B.Cu") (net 9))
 (segment (start 68.83 54.99) (end 66.8 54.99) (width 0.25) (layer "B.Cu") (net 9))
 (segment (start 71.65 57.81) (end 68.83 54.99) (width 0.25) (layer "B.Cu") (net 9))
 (segment (start 70.741589 63.701589) (end 71.65 62.793178) (width 0.25) (layer "B.Cu") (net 9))
 (segment (start 71.65 62.793178) (end 71.65 57.81) (width 0.25) (layer "B.Cu") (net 9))
 (segment (start 68.45 62.54) (end 68.87 62.54) (width 0.25) (layer "F.Cu") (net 1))
 (segment (start 65.4125 59.2125) (end 67.1 60.9) (width 0.25) (layer "F.Cu") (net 1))
 (segment (start 67.1 60.9) (end 67.1 63.475) (width 0.25) (layer "F.Cu") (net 1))
 (segment (start 62.7 59.2125) (end 65.4125 59.2125) (width 0.25) (layer "F.Cu") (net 1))
 (segment (start 67.515 63.475) (end 68.45 62.54) (width 0.25) (layer "F.Cu") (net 1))
 (segment (start 67.1 63.475) (end 67.515 63.475) (width 0.25) (layer "F.Cu") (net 1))
 (segment (start 62.08 61.99) (end 57.92 61.99) (width 0.25) (layer "F.Cu") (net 2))
 (segment (start 57.6 62.31) (end 57.6 63.225) (width 0.25) (layer "F.Cu") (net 2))
 (segment (start 57.92 61.99) (end 57.6 62.31) (width 0.25) (layer "F.Cu") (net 2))
 (segment (start 62.7 60.7875) (end 62.7 61.37) (width 0.25) (layer "F.Cu") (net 2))
 (segment (start 62.7 61.37) (end 62.08 61.99) (width 0.25) (layer "F.Cu") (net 2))
 (segment (start 64.825 63.475) (end 62.555 63.475) (width 0.25) (layer "F.Cu") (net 8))
 (segment (start 59.545 63.18) (end 59.5 63.225) (width 0.25) (layer "F.Cu") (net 8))
 (segment (start 62.26 63.18) (end 59.545 63.18) (width 0.25) (layer "F.Cu") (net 8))
 (segment (start 62.555 63.475) (end 62.26 63.18) (width 0.25) (layer "F.Cu") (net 8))
 (segment (start 67.1 66.84) (end 66.965 66.975) (width 0.25) (layer "F.Cu") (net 7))
 (segment (start 67.1 65.375) (end 67.1 66.69) (width 0.25) (layer "F.Cu") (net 7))
 (segment (start 67.1 66.69) (end 67.1 66.84) (width 0.25) (layer "F.Cu") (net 7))
 (segment (start 68.82 66.69) (end 68.88 66.63) (width 0.25) (layer "F.Cu") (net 7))
 (segment (start 66.965 66.975) (end 66.475 66.975) (width 0.25) (layer "F.Cu") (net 7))
 (segment (start 67.1 66.69) (end 68.82 66.69) (width 0.25) (layer "F.Cu") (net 7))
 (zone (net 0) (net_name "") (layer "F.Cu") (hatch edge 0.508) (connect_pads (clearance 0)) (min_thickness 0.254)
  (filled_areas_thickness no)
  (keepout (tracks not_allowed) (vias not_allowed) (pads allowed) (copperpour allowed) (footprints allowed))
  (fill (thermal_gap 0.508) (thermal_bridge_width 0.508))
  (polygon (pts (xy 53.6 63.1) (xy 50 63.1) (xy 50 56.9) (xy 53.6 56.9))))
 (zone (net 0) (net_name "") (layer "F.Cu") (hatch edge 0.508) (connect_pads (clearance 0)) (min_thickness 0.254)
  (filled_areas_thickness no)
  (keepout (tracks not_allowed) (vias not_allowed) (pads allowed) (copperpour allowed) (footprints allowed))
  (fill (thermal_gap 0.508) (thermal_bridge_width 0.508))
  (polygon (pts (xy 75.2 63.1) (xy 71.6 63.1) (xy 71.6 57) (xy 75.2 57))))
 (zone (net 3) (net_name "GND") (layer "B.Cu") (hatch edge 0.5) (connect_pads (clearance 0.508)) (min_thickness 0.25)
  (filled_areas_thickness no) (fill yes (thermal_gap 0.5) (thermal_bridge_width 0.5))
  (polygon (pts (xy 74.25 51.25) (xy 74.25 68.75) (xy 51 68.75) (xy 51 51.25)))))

